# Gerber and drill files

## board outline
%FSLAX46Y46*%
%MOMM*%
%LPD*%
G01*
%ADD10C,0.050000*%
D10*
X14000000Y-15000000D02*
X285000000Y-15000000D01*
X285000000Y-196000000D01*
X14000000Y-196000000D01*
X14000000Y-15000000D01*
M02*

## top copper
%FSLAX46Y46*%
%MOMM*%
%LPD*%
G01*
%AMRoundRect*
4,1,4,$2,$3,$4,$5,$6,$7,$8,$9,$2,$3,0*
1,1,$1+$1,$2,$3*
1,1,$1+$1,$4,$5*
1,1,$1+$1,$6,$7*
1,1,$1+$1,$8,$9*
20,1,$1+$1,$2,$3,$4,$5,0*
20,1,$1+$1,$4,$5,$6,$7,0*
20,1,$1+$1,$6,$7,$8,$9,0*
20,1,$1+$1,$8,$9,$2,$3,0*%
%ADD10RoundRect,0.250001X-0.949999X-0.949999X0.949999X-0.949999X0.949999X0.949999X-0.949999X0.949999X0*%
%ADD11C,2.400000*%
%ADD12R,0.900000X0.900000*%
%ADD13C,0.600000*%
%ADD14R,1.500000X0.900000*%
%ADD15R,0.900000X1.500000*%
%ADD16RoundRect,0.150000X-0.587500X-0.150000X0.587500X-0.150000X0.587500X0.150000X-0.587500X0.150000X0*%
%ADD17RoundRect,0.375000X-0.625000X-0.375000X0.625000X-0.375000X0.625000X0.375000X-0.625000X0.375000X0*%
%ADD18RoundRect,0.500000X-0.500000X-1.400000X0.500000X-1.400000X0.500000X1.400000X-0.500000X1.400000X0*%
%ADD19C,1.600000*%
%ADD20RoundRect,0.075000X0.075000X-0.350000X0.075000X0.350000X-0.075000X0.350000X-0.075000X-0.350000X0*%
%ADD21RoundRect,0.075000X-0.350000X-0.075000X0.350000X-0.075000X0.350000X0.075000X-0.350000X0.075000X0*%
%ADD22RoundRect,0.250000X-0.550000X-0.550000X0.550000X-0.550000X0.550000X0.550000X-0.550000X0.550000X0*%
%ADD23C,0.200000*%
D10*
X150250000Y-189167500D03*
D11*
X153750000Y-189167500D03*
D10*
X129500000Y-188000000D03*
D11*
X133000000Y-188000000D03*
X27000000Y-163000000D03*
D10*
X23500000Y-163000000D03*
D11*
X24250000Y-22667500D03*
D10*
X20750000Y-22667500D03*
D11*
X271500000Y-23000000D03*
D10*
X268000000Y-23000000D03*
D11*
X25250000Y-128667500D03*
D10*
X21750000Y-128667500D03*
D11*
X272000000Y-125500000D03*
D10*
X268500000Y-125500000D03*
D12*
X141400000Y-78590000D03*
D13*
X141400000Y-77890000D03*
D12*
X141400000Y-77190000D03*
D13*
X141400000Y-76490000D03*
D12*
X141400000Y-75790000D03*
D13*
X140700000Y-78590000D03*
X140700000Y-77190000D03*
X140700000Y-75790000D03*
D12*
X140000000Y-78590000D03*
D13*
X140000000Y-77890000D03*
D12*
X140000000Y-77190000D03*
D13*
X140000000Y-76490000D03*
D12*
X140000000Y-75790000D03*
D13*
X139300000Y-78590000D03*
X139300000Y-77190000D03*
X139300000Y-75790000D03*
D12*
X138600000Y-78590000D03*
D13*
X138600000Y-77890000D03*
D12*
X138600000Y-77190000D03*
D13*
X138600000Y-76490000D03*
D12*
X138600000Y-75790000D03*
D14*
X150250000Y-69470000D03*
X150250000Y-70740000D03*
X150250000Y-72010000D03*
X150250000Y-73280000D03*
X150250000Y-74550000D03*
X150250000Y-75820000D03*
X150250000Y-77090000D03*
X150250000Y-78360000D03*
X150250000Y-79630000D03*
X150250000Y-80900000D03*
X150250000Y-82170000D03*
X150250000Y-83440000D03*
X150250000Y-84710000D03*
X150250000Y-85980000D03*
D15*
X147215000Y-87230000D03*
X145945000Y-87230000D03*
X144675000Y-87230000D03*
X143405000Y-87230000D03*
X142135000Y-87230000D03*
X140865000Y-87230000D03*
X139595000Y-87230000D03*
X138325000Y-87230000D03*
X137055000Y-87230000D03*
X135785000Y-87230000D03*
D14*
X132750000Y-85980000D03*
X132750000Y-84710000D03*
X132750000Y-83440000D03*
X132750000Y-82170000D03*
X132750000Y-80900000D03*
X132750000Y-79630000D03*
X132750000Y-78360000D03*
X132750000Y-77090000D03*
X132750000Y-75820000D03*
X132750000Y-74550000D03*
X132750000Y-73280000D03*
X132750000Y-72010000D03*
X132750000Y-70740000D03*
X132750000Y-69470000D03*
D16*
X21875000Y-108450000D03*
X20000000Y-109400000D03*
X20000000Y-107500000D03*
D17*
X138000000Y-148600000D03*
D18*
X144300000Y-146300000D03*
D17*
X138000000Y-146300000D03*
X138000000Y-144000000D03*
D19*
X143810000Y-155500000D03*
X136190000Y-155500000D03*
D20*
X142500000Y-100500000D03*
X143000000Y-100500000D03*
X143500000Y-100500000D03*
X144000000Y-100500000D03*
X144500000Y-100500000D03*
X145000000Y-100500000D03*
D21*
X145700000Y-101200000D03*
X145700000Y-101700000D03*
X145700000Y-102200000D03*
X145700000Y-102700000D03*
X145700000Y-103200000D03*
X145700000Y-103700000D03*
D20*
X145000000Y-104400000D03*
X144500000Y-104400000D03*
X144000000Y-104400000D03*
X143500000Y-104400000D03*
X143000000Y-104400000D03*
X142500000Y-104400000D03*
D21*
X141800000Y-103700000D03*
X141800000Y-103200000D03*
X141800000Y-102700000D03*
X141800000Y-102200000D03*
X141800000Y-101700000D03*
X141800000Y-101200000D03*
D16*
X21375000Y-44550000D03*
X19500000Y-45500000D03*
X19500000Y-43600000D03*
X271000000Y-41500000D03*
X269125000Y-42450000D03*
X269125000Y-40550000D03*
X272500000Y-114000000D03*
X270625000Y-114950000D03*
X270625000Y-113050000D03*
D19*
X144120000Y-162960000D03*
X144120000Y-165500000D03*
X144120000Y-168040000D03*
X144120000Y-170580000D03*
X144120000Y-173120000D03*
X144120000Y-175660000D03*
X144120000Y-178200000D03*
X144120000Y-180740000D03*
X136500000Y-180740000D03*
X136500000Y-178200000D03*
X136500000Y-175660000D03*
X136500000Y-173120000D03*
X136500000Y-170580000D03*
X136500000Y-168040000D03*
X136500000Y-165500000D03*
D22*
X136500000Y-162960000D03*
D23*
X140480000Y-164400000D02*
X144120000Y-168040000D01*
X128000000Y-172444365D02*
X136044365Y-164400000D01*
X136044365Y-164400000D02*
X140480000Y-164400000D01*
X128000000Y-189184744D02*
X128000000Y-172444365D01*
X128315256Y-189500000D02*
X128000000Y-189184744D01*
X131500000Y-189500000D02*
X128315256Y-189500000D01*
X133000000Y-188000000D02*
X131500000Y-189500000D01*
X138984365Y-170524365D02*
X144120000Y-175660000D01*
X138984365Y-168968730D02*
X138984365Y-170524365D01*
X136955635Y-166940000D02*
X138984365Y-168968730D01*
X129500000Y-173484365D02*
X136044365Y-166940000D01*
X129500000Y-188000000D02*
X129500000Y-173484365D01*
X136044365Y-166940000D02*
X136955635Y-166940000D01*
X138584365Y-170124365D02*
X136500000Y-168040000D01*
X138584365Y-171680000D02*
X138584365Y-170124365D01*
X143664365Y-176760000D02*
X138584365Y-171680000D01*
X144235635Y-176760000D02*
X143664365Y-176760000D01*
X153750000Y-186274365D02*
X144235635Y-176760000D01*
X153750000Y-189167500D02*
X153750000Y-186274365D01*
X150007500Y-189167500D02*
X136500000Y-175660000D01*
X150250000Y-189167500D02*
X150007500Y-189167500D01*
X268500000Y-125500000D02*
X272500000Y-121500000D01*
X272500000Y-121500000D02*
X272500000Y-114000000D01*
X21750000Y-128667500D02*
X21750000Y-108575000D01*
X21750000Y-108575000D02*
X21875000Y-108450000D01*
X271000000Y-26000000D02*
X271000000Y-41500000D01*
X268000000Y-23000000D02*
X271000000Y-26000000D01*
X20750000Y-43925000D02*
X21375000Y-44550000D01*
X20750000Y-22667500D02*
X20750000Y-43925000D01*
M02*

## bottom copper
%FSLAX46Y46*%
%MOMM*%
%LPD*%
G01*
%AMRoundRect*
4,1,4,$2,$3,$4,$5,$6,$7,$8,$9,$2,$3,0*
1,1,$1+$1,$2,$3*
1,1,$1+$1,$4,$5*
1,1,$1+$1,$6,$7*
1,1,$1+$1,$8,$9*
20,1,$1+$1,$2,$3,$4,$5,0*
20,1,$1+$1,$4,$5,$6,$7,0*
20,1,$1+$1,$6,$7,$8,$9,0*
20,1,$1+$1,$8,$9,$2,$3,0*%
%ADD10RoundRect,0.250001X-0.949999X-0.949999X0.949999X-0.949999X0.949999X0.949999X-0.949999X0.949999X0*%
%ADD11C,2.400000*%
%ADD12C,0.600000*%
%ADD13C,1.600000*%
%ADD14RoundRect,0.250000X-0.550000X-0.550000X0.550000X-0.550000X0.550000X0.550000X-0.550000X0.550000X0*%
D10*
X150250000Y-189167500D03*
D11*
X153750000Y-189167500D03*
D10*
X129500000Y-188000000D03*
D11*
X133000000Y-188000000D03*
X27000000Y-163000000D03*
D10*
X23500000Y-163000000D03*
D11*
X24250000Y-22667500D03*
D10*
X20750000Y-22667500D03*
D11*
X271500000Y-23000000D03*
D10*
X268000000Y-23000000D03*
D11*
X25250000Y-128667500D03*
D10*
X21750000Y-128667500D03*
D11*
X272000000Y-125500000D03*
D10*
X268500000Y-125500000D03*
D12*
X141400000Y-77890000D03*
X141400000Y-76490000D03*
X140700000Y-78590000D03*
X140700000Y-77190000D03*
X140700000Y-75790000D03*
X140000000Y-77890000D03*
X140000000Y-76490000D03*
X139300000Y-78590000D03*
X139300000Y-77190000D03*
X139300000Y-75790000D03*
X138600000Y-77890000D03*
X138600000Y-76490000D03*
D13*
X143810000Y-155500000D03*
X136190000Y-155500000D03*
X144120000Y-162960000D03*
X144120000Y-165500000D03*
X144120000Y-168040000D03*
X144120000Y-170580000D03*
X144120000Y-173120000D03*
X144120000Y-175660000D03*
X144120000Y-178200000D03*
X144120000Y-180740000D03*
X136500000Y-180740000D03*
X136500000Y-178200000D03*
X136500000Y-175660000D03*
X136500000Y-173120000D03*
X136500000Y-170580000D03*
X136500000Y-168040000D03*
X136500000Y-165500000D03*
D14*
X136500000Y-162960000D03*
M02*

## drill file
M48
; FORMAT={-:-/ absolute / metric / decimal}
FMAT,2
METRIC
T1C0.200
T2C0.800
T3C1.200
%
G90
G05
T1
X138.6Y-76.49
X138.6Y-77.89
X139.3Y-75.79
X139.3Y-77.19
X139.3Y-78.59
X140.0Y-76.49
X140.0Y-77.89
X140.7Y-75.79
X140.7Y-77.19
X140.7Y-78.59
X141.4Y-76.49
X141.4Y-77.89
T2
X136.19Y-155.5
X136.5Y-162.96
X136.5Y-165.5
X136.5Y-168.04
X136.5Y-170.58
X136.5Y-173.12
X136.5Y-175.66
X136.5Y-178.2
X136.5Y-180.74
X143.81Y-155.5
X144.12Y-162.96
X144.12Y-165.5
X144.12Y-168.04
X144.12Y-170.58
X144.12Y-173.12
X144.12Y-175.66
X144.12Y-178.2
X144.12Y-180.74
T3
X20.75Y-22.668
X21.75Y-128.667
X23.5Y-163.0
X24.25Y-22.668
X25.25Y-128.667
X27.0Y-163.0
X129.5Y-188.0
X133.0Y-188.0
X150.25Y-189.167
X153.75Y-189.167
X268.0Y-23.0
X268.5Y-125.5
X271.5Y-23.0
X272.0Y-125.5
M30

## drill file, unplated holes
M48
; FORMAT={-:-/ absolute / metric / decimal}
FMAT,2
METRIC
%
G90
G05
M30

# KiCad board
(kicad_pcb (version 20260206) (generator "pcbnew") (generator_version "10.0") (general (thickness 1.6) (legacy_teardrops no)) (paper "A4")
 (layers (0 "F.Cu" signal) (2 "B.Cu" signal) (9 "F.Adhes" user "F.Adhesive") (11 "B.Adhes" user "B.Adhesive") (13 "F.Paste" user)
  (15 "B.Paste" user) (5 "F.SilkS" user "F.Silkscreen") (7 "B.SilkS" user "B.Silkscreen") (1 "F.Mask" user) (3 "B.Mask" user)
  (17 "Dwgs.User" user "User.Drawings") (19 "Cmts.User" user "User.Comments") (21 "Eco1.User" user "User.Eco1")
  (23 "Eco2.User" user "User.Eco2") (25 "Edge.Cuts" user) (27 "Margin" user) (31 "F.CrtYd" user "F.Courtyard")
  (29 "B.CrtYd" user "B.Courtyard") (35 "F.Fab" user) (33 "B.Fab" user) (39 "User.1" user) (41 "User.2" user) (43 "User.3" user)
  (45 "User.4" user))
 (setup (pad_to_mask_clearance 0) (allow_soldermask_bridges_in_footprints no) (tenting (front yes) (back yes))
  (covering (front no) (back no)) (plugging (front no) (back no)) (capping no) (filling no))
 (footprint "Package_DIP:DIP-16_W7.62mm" (layer "F.Cu") (at 136.5 162.96)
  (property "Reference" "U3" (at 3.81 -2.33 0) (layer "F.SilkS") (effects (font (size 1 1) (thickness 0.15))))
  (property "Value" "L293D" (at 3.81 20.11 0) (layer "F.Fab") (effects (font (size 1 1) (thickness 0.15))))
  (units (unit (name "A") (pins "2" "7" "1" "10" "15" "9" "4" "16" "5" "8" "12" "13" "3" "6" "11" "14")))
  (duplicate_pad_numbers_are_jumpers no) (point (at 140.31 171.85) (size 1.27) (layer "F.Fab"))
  (pad "1" thru_hole roundrect (at 0 0) (size 1.6 1.6) (drill 0.8) (layers "*.Cu" "*.Mask") (remove_unused_layers no)
   (roundrect_rratio 0.15625) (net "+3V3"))
  (pad "2" thru_hole circle (at 0 2.54) (size 1.6 1.6) (drill 0.8) (layers "*.Cu" "*.Mask") (remove_unused_layers no) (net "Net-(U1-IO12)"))
  (pad "3" thru_hole circle (at 0 5.08) (size 1.6 1.6) (drill 0.8) (layers "*.Cu" "*.Mask") (remove_unused_layers no) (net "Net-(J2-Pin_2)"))
  (pad "4" thru_hole circle (at 0 7.62) (size 1.6 1.6) (drill 0.8) (layers "*.Cu" "*.Mask") (remove_unused_layers no) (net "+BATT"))
  (pad "5" thru_hole circle (at 0 10.16) (size 1.6 1.6) (drill 0.8) (layers "*.Cu" "*.Mask") (remove_unused_layers no) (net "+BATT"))
  (pad "6" thru_hole circle (at 0 12.7) (size 1.6 1.6) (drill 0.8) (layers "*.Cu" "*.Mask") (remove_unused_layers no) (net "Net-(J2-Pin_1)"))
  (pad "7" thru_hole circle (at 0 15.24) (size 1.6 1.6) (drill 0.8) (layers "*.Cu" "*.Mask") (remove_unused_layers no) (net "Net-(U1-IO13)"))
  (pad "8" thru_hole circle (at 0 17.78) (size 1.6 1.6) (drill 0.8) (layers "*.Cu" "*.Mask") (remove_unused_layers no) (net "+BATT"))
  (pad "9" thru_hole circle (at 7.62 17.78) (size 1.6 1.6) (drill 0.8) (layers "*.Cu" "*.Mask") (remove_unused_layers no) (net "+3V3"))
  (pad "10" thru_hole circle (at 7.62 15.24) (size 1.6 1.6) (drill 0.8) (layers "*.Cu" "*.Mask") (remove_unused_layers no)
   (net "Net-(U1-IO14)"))
  (pad "11" thru_hole circle (at 7.62 12.7) (size 1.6 1.6) (drill 0.8) (layers "*.Cu" "*.Mask") (remove_unused_layers no)
   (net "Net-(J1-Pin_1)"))
  (pad "12" thru_hole circle (at 7.62 10.16) (size 1.6 1.6) (drill 0.8) (layers "*.Cu" "*.Mask") (remove_unused_layers no) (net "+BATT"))
  (pad "13" thru_hole circle (at 7.62 7.62) (size 1.6 1.6) (drill 0.8) (layers "*.Cu" "*.Mask") (remove_unused_layers no) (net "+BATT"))
  (pad "14" thru_hole circle (at 7.62 5.08) (size 1.6 1.6) (drill 0.8) (layers "*.Cu" "*.Mask") (remove_unused_layers no)
   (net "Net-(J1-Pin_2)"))
  (pad "15" thru_hole circle (at 7.62 2.54) (size 1.6 1.6) (drill 0.8) (layers "*.Cu" "*.Mask") (remove_unused_layers no)
   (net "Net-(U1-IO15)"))
  (pad "16" thru_hole circle (at 7.62 0) (size 1.6 1.6) (drill 0.8) (layers "*.Cu" "*.Mask") (remove_unused_layers no)
   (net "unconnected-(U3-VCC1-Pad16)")))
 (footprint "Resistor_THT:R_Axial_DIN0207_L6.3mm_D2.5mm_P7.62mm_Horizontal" (layer "F.Cu") (at 136.19 155.5)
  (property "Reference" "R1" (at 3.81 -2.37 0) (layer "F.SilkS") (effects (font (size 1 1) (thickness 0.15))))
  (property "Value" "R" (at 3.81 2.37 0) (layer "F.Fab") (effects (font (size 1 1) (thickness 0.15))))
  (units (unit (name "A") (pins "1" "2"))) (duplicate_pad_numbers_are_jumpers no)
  (pad "1" thru_hole circle (at 0 0) (size 1.6 1.6) (drill 0.8) (layers "*.Cu" "*.Mask") (remove_unused_layers no) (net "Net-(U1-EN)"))
  (pad "2" thru_hole circle (at 7.62 0) (size 1.6 1.6) (drill 0.8) (layers "*.Cu" "*.Mask") (remove_unused_layers no) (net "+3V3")))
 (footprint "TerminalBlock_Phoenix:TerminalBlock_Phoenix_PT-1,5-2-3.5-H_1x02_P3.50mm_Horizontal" (layer "F.Cu") (at 268.5 125.5)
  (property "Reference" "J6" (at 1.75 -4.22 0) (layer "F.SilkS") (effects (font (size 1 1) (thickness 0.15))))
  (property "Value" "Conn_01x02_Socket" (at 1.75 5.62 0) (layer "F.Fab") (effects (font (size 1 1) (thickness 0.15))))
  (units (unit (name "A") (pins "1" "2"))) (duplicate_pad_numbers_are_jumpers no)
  (pad "1" thru_hole roundrect (at 0 0) (size 2.4 2.4) (drill 1.2) (layers "*.Cu" "*.Mask") (remove_unused_layers no)
   (roundrect_rratio 0.104167) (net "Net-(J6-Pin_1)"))
  (pad "2" thru_hole circle (at 3.5 0) (size 2.4 2.4) (drill 1.2) (layers "*.Cu" "*.Mask") (remove_unused_layers no) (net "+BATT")))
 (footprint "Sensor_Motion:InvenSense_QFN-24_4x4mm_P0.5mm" (layer "F.Cu") (at 143.75 102.45)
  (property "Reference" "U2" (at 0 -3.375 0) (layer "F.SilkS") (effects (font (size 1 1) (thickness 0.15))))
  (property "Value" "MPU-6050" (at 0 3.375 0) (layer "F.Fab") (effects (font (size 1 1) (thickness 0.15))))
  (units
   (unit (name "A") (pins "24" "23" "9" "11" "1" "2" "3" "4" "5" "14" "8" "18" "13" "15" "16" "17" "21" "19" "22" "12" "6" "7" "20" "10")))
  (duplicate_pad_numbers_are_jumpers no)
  (pad "1" smd roundrect (at -1.95 -1.25) (size 0.85 0.3) (layers "F.Cu" "F.Mask" "F.Paste") (roundrect_rratio 0.25)
   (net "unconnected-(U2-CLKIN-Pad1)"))
  (pad "2" smd roundrect (at -1.95 -0.75) (size 0.85 0.3) (layers "F.Cu" "F.Mask" "F.Paste") (roundrect_rratio 0.25)
   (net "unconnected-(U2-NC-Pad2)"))
  (pad "3" smd roundrect (at -1.95 -0.25) (size 0.85 0.3) (layers "F.Cu" "F.Mask" "F.Paste") (roundrect_rratio 0.25)
   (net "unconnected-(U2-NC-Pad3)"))
  (pad "4" smd roundrect (at -1.95 0.25) (size 0.85 0.3) (layers "F.Cu" "F.Mask" "F.Paste") (roundrect_rratio 0.25)
   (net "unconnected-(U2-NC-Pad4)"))
  (pad "5" smd roundrect (at -1.95 0.75) (size 0.85 0.3) (layers "F.Cu" "F.Mask" "F.Paste") (roundrect_rratio 0.25)
   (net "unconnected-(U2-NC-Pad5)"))
  (pad "6" smd roundrect (at -1.95 1.25) (size 0.85 0.3) (layers "F.Cu" "F.Mask" "F.Paste") (roundrect_rratio 0.25)
   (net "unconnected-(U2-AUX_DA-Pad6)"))
  (pad "7" smd roundrect (at -1.25 1.95 90) (size 0.85 0.3) (layers "F.Cu" "F.Mask" "F.Paste") (roundrect_rratio 0.25)
   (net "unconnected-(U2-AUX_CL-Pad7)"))
  (pad "8" smd roundrect (at -0.75 1.95 90) (size 0.85 0.3) (layers "F.Cu" "F.Mask" "F.Paste") (roundrect_rratio 0.25) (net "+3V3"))
  (pad "9" smd roundrect (at -0.25 1.95 90) (size 0.85 0.3) (layers "F.Cu" "F.Mask" "F.Paste") (roundrect_rratio 0.25)
   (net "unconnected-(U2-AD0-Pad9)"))
  (pad "10" smd roundrect (at 0.25 1.95 90) (size 0.85 0.3) (layers "F.Cu" "F.Mask" "F.Paste") (roundrect_rratio 0.25)
   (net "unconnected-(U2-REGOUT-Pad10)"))
  (pad "11" smd roundrect (at 0.75 1.95 90) (size 0.85 0.3) (layers "F.Cu" "F.Mask" "F.Paste") (roundrect_rratio 0.25)
   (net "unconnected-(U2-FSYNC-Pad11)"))
  (pad "12" smd roundrect (at 1.25 1.95 90) (size 0.85 0.3) (layers "F.Cu" "F.Mask" "F.Paste") (roundrect_rratio 0.25)
   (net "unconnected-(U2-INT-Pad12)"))
  (pad "13" smd roundrect (at 1.95 1.25) (size 0.85 0.3) (layers "F.Cu" "F.Mask" "F.Paste") (roundrect_rratio 0.25) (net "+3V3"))
  (pad "14" smd roundrect (at 1.95 0.75) (size 0.85 0.3) (layers "F.Cu" "F.Mask" "F.Paste") (roundrect_rratio 0.25)
   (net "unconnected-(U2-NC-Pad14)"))
  (pad "15" smd roundrect (at 1.95 0.25) (size 0.85 0.3) (layers "F.Cu" "F.Mask" "F.Paste") (roundrect_rratio 0.25)
   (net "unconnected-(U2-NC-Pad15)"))
  (pad "16" smd roundrect (at 1.95 -0.25) (size 0.85 0.3) (layers "F.Cu" "F.Mask" "F.Paste") (roundrect_rratio 0.25)
   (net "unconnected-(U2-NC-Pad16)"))
  (pad "17" smd roundrect (at 1.95 -0.75) (size 0.85 0.3) (layers "F.Cu" "F.Mask" "F.Paste") (roundrect_rratio 0.25)
   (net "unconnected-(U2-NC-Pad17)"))
  (pad "18" smd roundrect (at 1.95 -1.25) (size 0.85 0.3) (layers "F.Cu" "F.Mask" "F.Paste") (roundrect_rratio 0.25) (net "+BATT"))
  (pad "19" smd roundrect (at 1.25 -1.95 90) (size 0.85 0.3) (layers "F.Cu" "F.Mask" "F.Paste") (roundrect_rratio 0.25)
   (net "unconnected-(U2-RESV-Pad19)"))
  (pad "20" smd roundrect (at 0.75 -1.95 90) (size 0.85 0.3) (layers "F.Cu" "F.Mask" "F.Paste") (roundrect_rratio 0.25)
   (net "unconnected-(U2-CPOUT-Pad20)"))
  (pad "21" smd roundrect (at 0.25 -1.95 90) (size 0.85 0.3) (layers "F.Cu" "F.Mask" "F.Paste") (roundrect_rratio 0.25)
   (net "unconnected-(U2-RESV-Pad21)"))
  (pad "22" smd roundrect (at -0.25 -1.95 90) (size 0.85 0.3) (layers "F.Cu" "F.Mask" "F.Paste") (roundrect_rratio 0.25)
   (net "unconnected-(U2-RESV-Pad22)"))
  (pad "23" smd roundrect (at -0.75 -1.95 90) (size 0.85 0.3) (layers "F.Cu" "F.Mask" "F.Paste") (roundrect_rratio 0.25)
   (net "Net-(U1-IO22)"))
  (pad "24" smd roundrect (at -1.25 -1.95 90) (size 0.85 0.3) (layers "F.Cu" "F.Mask" "F.Paste") (roundrect_rratio 0.25)
   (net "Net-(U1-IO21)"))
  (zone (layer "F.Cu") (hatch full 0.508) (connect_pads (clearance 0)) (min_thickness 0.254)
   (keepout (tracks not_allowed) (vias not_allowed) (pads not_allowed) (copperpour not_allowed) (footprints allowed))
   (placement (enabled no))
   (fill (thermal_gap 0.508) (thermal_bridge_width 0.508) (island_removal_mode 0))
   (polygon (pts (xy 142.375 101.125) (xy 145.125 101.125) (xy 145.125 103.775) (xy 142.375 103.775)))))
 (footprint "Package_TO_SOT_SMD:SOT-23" (layer "F.Cu") (at 20.4375 44.55)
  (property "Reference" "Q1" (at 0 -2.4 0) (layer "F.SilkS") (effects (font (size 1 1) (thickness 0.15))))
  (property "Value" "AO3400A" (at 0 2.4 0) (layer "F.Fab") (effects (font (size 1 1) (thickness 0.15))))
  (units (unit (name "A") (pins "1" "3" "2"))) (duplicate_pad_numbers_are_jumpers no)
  (pad "1" smd roundrect (at -0.9375 -0.95) (size 1.475 0.6) (layers "F.Cu" "F.Mask" "F.Paste") (roundrect_rratio 0.25) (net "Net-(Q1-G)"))
  (pad "2" smd roundrect (at -0.9375 0.95) (size 1.475 0.6) (layers "F.Cu" "F.Mask" "F.Paste") (roundrect_rratio 0.25)
   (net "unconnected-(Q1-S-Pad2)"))
  (pad "3" smd roundrect (at 0.9375 0) (size 1.475 0.6) (layers "F.Cu" "F.Mask" "F.Paste") (roundrect_rratio 0.25) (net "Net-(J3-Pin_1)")))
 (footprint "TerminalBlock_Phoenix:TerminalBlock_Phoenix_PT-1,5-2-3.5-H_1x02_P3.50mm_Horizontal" (layer "F.Cu") (at 150.25 189.1675)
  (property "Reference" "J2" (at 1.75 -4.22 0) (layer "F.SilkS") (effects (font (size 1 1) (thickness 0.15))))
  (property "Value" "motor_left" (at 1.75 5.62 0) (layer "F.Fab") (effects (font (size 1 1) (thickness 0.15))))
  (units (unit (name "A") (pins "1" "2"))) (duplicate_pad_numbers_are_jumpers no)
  (pad "1" thru_hole roundrect (at 0 0) (size 2.4 2.4) (drill 1.2) (layers "*.Cu" "*.Mask") (remove_unused_layers no)
   (roundrect_rratio 0.104167) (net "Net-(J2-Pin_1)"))
  (pad "2" thru_hole circle (at 3.5 0) (size 2.4 2.4) (drill 1.2) (layers "*.Cu" "*.Mask") (remove_unused_layers no) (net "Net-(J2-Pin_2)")))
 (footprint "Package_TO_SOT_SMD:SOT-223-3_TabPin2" (layer "F.Cu") (at 141.15 146.3)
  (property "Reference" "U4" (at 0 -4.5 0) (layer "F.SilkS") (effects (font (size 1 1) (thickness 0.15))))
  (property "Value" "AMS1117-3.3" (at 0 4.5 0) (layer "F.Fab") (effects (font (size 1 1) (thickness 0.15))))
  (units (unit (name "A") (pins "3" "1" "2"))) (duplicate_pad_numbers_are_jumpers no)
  (pad "1" smd roundrect (at -3.15 -2.3) (size 2 1.5) (layers "F.Cu" "F.Mask" "F.Paste") (roundrect_rratio 0.25) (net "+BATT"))
  (pad "2" smd roundrect (at -3.15 0) (size 2 1.5) (layers "F.Cu" "F.Mask" "F.Paste") (roundrect_rratio 0.25) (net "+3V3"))
  (pad "2" smd roundrect (at 3.15 0) (size 2 3.8) (layers "F.Cu" "F.Mask" "F.Paste") (roundrect_rratio 0.25) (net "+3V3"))
  (pad "3" smd roundrect (at -3.15 2.3) (size 2 1.5) (layers "F.Cu" "F.Mask" "F.Paste") (roundrect_rratio 0.25) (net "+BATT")))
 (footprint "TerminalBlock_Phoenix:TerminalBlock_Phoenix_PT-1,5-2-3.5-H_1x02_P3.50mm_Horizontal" (layer "F.Cu") (at 23.5 163)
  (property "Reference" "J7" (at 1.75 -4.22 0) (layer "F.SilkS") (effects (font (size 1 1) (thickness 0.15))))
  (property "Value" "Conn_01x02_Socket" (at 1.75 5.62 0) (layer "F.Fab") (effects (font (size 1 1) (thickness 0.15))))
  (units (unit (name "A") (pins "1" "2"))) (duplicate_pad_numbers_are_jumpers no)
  (pad "1" thru_hole roundrect (at 0 0) (size 2.4 2.4) (drill 1.2) (layers "*.Cu" "*.Mask") (remove_unused_layers no)
   (roundrect_rratio 0.104167) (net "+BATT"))
  (pad "2" thru_hole circle (at 3.5 0) (size 2.4 2.4) (drill 1.2) (layers "*.Cu" "*.Mask") (remove_unused_layers no) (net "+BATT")))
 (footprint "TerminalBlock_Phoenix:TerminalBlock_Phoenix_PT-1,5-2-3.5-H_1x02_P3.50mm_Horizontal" (layer "F.Cu") (at 21.75 128.6675)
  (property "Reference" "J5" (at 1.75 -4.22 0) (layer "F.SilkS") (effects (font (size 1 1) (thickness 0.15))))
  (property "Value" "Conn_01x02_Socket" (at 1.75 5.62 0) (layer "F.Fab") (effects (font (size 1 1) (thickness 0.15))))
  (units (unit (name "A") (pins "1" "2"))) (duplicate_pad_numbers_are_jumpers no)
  (pad "1" thru_hole roundrect (at 0 0) (size 2.4 2.4) (drill 1.2) (layers "*.Cu" "*.Mask") (remove_unused_layers no)
   (roundrect_rratio 0.104167) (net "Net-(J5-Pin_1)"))
  (pad "2" thru_hole circle (at 3.5 0) (size 2.4 2.4) (drill 1.2) (layers "*.Cu" "*.Mask") (remove_unused_layers no) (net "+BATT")))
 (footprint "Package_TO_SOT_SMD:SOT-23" (layer "F.Cu") (at 20.9375 108.45)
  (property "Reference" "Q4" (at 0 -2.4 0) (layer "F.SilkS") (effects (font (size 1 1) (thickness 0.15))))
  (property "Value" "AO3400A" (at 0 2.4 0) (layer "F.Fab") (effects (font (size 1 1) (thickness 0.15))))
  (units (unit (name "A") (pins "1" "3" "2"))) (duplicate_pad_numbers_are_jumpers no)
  (pad "1" smd roundrect (at -0.9375 -0.95) (size 1.475 0.6) (layers "F.Cu" "F.Mask" "F.Paste") (roundrect_rratio 0.25) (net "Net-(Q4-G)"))
  (pad "2" smd roundrect (at -0.9375 0.95) (size 1.475 0.6) (layers "F.Cu" "F.Mask" "F.Paste") (roundrect_rratio 0.25)
   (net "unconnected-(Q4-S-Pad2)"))
  (pad "3" smd roundrect (at 0.9375 0) (size 1.475 0.6) (layers "F.Cu" "F.Mask" "F.Paste") (roundrect_rratio 0.25) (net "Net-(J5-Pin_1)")))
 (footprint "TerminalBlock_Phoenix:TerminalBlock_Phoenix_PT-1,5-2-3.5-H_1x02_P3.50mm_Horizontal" (layer "F.Cu") (at 268 23)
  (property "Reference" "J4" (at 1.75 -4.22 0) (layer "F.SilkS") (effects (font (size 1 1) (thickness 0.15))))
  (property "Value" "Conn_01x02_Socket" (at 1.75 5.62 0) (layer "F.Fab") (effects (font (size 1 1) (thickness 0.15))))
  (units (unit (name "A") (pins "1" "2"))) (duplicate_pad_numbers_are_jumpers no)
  (pad "1" thru_hole roundrect (at 0 0) (size 2.4 2.4) (drill 1.2) (layers "*.Cu" "*.Mask") (remove_unused_layers no)
   (roundrect_rratio 0.104167) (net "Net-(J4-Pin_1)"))
  (pad "2" thru_hole circle (at 3.5 0) (size 2.4 2.4) (drill 1.2) (layers "*.Cu" "*.Mask") (remove_unused_layers no) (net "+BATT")))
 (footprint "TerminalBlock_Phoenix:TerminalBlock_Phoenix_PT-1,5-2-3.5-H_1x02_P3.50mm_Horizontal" (layer "F.Cu") (at 129.5 188)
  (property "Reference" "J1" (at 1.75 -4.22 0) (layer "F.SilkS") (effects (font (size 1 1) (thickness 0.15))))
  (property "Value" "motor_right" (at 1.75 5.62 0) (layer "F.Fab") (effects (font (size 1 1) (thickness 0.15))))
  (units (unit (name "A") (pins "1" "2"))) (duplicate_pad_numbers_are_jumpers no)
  (pad "1" thru_hole roundrect (at 0 0) (size 2.4 2.4) (drill 1.2) (layers "*.Cu" "*.Mask") (remove_unused_layers no)
   (roundrect_rratio 0.104167) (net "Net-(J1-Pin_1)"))
  (pad "2" thru_hole circle (at 3.5 0) (size 2.4 2.4) (drill 1.2) (layers "*.Cu" "*.Mask") (remove_unused_layers no) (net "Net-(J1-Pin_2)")))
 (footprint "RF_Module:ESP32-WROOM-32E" (layer "F.Cu") (at 141.5 74.73)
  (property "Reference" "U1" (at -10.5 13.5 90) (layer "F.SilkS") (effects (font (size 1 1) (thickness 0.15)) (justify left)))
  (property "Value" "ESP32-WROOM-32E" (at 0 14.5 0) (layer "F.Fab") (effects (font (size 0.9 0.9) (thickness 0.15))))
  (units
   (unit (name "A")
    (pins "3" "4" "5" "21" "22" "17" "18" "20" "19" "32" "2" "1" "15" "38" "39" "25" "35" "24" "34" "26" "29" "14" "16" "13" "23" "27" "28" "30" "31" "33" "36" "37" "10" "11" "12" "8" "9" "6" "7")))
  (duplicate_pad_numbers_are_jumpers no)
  (pad "1" smd rect (at -8.75 -5.26) (size 1.5 0.9) (layers "F.Cu" "F.Mask" "F.Paste") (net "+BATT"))
  (pad "2" smd rect (at -8.75 -3.99) (size 1.5 0.9) (layers "F.Cu" "F.Mask" "F.Paste") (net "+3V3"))
  (pad "3" smd rect (at -8.75 -2.72) (size 1.5 0.9) (layers "F.Cu" "F.Mask" "F.Paste") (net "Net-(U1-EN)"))
  (pad "4" smd rect (at -8.75 -1.45) (size 1.5 0.9) (layers "F.Cu" "F.Mask" "F.Paste") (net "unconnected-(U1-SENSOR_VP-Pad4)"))
  (pad "5" smd rect (at -8.75 -0.18) (size 1.5 0.9) (layers "F.Cu" "F.Mask" "F.Paste") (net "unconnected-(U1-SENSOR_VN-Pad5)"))
  (pad "6" smd rect (at -8.75 1.09) (size 1.5 0.9) (layers "F.Cu" "F.Mask" "F.Paste") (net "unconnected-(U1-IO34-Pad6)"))
  (pad "7" smd rect (at -8.75 2.36) (size 1.5 0.9) (layers "F.Cu" "F.Mask" "F.Paste") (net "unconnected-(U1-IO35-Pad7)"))
  (pad "8" smd rect (at -8.75 3.63) (size 1.5 0.9) (layers "F.Cu" "F.Mask" "F.Paste") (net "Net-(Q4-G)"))
  (pad "9" smd rect (at -8.75 4.9) (size 1.5 0.9) (layers "F.Cu" "F.Mask" "F.Paste") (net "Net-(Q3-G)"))
  (pad "10" smd rect (at -8.75 6.17) (size 1.5 0.9) (layers "F.Cu" "F.Mask" "F.Paste") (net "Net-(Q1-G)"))
  (pad "11" smd rect (at -8.75 7.44) (size 1.5 0.9) (layers "F.Cu" "F.Mask" "F.Paste") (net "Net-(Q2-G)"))
  (pad "12" smd rect (at -8.75 8.71) (size 1.5 0.9) (layers "F.Cu" "F.Mask" "F.Paste") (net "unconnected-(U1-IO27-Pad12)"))
  (pad "13" smd rect (at -8.75 9.98) (size 1.5 0.9) (layers "F.Cu" "F.Mask" "F.Paste") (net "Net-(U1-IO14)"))
  (pad "14" smd rect (at -8.75 11.25) (size 1.5 0.9) (layers "F.Cu" "F.Mask" "F.Paste") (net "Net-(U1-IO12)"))
  (pad "15" smd rect (at -5.715 12.5 90) (size 1.5 0.9) (layers "F.Cu" "F.Mask" "F.Paste") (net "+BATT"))
  (pad "16" smd rect (at -4.445 12.5 90) (size 1.5 0.9) (layers "F.Cu" "F.Mask" "F.Paste") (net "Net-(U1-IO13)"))
  (pad "17" smd rect (at -3.175 12.5 90) (size 1.5 0.9) (layers "F.Cu" "F.Mask" "F.Paste") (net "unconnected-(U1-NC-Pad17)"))
  (pad "18" smd rect (at -1.905 12.5 90) (size 1.5 0.9) (layers "F.Cu" "F.Mask" "F.Paste") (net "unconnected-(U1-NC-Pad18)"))
  (pad "19" smd rect (at -0.635 12.5 90) (size 1.5 0.9) (layers "F.Cu" "F.Mask" "F.Paste") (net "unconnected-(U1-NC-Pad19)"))
  (pad "20" smd rect (at 0.635 12.5 90) (size 1.5 0.9) (layers "F.Cu" "F.Mask" "F.Paste") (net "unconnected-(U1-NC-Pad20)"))
  (pad "21" smd rect (at 1.905 12.5 90) (size 1.5 0.9) (layers "F.Cu" "F.Mask" "F.Paste") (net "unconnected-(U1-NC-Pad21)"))
  (pad "22" smd rect (at 3.175 12.5 90) (size 1.5 0.9) (layers "F.Cu" "F.Mask" "F.Paste") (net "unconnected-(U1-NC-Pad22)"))
  (pad "23" smd rect (at 4.445 12.5 90) (size 1.5 0.9) (layers "F.Cu" "F.Mask" "F.Paste") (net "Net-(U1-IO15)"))
  (pad "24" smd rect (at 5.715 12.5 90) (size 1.5 0.9) (layers "F.Cu" "F.Mask" "F.Paste") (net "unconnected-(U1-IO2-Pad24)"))
  (pad "25" smd rect (at 8.75 11.25) (size 1.5 0.9) (layers "F.Cu" "F.Mask" "F.Paste") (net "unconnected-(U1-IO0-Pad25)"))
  (pad "26" smd rect (at 8.75 9.98) (size 1.5 0.9) (layers "F.Cu" "F.Mask" "F.Paste") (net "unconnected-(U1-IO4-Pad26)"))
  (pad "27" smd rect (at 8.75 8.71) (size 1.5 0.9) (layers "F.Cu" "F.Mask" "F.Paste") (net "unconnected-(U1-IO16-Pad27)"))
  (pad "28" smd rect (at 8.75 7.44) (size 1.5 0.9) (layers "F.Cu" "F.Mask" "F.Paste") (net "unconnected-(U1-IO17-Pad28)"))
  (pad "29" smd rect (at 8.75 6.17) (size 1.5 0.9) (layers "F.Cu" "F.Mask" "F.Paste") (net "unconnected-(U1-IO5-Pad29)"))
  (pad "30" smd rect (at 8.75 4.9) (size 1.5 0.9) (layers "F.Cu" "F.Mask" "F.Paste") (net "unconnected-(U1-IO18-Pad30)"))
  (pad "31" smd rect (at 8.75 3.63) (size 1.5 0.9) (layers "F.Cu" "F.Mask" "F.Paste") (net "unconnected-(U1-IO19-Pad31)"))
  (pad "32" smd rect (at 8.75 2.36) (size 1.5 0.9) (layers "F.Cu" "F.Mask" "F.Paste") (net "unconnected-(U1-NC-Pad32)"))
  (pad "33" smd rect (at 8.75 1.09) (size 1.5 0.9) (layers "F.Cu" "F.Mask" "F.Paste") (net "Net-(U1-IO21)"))
  (pad "34" smd rect (at 8.75 -0.18) (size 1.5 0.9) (layers "F.Cu" "F.Mask" "F.Paste") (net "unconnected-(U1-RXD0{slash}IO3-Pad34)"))
  (pad "35" smd rect (at 8.75 -1.45) (size 1.5 0.9) (layers "F.Cu" "F.Mask" "F.Paste") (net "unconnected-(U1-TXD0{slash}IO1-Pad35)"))
  (pad "36" smd rect (at 8.75 -2.72) (size 1.5 0.9) (layers "F.Cu" "F.Mask" "F.Paste") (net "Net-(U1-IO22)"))
  (pad "37" smd rect (at 8.75 -3.99) (size 1.5 0.9) (layers "F.Cu" "F.Mask" "F.Paste") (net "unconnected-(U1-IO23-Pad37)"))
  (pad "38" smd rect (at 8.75 -5.26) (size 1.5 0.9) (layers "F.Cu" "F.Mask" "F.Paste") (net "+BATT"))
  (pad "39" smd rect (at -2.9 1.06) (size 0.9 0.9) (layers "F.Cu" "F.Mask" "F.Paste") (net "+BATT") (zone_connect 2))
  (pad "39" thru_hole circle (at -2.9 1.76) (size 0.6 0.6) (drill 0.2) (layers "*.Cu" "*.Mask") (remove_unused_layers no) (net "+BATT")
   (zone_connect 2))
  (pad "39" smd rect (at -2.9 2.46) (size 0.9 0.9) (layers "F.Cu" "F.Mask" "F.Paste") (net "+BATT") (zone_connect 2))
  (pad "39" thru_hole circle (at -2.9 3.16) (size 0.6 0.6) (drill 0.2) (layers "*.Cu" "*.Mask") (remove_unused_layers no) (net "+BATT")
   (zone_connect 2))
  (pad "39" smd rect (at -2.9 3.86) (size 0.9 0.9) (layers "F.Cu" "F.Mask" "F.Paste") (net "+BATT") (zone_connect 2))
  (pad "39" thru_hole circle (at -2.2 1.06) (size 0.6 0.6) (drill 0.2) (layers "*.Cu" "*.Mask") (remove_unused_layers no) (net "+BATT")
   (zone_connect 2))
  (pad "39" thru_hole circle (at -2.2 2.46) (size 0.6 0.6) (drill 0.2) (layers "*.Cu" "*.Mask") (remove_unused_layers no) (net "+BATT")
   (zone_connect 2))
  (pad "39" thru_hole circle (at -2.2 3.86) (size 0.6 0.6) (drill 0.2) (layers "*.Cu" "*.Mask") (remove_unused_layers no) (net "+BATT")
   (zone_connect 2))
  (pad "39" smd rect (at -1.5 1.06) (size 0.9 0.9) (layers "F.Cu" "F.Mask" "F.Paste") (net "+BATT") (zone_connect 2))
  (pad "39" thru_hole circle (at -1.5 1.76) (size 0.6 0.6) (drill 0.2) (layers "*.Cu" "*.Mask") (remove_unused_layers no) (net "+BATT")
   (zone_connect 2))
  (pad "39" smd rect (at -1.5 2.46) (size 0.9 0.9) (layers "F.Cu" "F.Mask" "F.Paste") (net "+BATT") (zone_connect 2))
  (pad "39" thru_hole circle (at -1.5 3.16) (size 0.6 0.6) (drill 0.2) (layers "*.Cu" "*.Mask") (remove_unused_layers no) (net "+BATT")
   (zone_connect 2))
  (pad "39" smd rect (at -1.5 3.86) (size 0.9 0.9) (layers "F.Cu" "F.Mask" "F.Paste") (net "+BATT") (zone_connect 2))
  (pad "39" thru_hole circle (at -0.8 1.06) (size 0.6 0.6) (drill 0.2) (layers "*.Cu" "*.Mask") (remove_unused_layers no) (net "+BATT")
   (zone_connect 2))
  (pad "39" thru_hole circle (at -0.8 2.46) (size 0.6 0.6) (drill 0.2) (layers "*.Cu" "*.Mask") (remove_unused_layers no) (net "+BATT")
   (zone_connect 2))
  (pad "39" thru_hole circle (at -0.8 3.86) (size 0.6 0.6) (drill 0.2) (layers "*.Cu" "*.Mask") (remove_unused_layers no) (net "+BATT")
   (zone_connect 2))
  (pad "39" smd rect (at -0.1 1.06) (size 0.9 0.9) (layers "F.Cu" "F.Mask" "F.Paste") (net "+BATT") (zone_connect 2))
  (pad "39" thru_hole circle (at -0.1 1.76) (size 0.6 0.6) (drill 0.2) (layers "*.Cu" "*.Mask") (remove_unused_layers no) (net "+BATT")
   (zone_connect 2))
  (pad "39" smd rect (at -0.1 2.46) (size 0.9 0.9) (layers "F.Cu" "F.Mask" "F.Paste") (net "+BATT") (zone_connect 2))
  (pad "39" thru_hole circle (at -0.1 3.16) (size 0.6 0.6) (drill 0.2) (layers "*.Cu" "*.Mask") (remove_unused_layers no) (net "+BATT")
   (zone_connect 2))
  (pad "39" smd rect (at -0.1 3.86) (size 0.9 0.9) (layers "F.Cu" "F.Mask" "F.Paste") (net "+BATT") (zone_connect 2))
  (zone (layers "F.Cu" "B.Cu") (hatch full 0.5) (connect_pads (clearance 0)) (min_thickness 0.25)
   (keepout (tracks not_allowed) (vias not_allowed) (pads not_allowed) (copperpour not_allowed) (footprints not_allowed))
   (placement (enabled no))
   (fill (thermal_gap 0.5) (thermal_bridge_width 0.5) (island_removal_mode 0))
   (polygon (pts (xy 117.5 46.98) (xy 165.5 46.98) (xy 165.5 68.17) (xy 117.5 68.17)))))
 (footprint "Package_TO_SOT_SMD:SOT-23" (layer "F.Cu") (at 271.5625 114)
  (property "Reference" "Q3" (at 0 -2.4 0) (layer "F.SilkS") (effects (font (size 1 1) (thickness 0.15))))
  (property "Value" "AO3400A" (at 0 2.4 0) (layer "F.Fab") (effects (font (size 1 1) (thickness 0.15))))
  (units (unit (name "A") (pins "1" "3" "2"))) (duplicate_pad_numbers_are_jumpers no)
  (pad "1" smd roundrect (at -0.9375 -0.95) (size 1.475 0.6) (layers "F.Cu" "F.Mask" "F.Paste") (roundrect_rratio 0.25) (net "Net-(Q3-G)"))
  (pad "2" smd roundrect (at -0.9375 0.95) (size 1.475 0.6) (layers "F.Cu" "F.Mask" "F.Paste") (roundrect_rratio 0.25)
   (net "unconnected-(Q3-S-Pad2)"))
  (pad "3" smd roundrect (at 0.9375 0) (size 1.475 0.6) (layers "F.Cu" "F.Mask" "F.Paste") (roundrect_rratio 0.25) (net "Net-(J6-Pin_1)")))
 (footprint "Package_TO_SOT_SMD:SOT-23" (layer "F.Cu") (at 270.0625 41.5)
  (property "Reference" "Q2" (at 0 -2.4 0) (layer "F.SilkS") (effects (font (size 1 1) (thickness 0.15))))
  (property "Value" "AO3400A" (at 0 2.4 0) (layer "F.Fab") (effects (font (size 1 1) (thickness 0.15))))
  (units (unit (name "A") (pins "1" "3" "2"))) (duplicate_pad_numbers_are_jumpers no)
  (pad "1" smd roundrect (at -0.9375 -0.95) (size 1.475 0.6) (layers "F.Cu" "F.Mask" "F.Paste") (roundrect_rratio 0.25) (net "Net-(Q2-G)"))
  (pad "2" smd roundrect (at -0.9375 0.95) (size 1.475 0.6) (layers "F.Cu" "F.Mask" "F.Paste") (roundrect_rratio 0.25)
   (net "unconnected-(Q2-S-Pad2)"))
  (pad "3" smd roundrect (at 0.9375 0) (size 1.475 0.6) (layers "F.Cu" "F.Mask" "F.Paste") (roundrect_rratio 0.25) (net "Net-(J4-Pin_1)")))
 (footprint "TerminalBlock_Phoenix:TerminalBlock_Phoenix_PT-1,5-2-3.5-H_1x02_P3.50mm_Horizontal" (layer "F.Cu") (at 20.75 22.6675)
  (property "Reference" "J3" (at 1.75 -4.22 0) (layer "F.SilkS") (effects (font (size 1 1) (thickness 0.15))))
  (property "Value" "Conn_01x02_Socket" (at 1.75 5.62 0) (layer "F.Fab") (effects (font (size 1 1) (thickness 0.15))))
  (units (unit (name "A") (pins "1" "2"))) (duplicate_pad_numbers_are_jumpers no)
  (pad "1" thru_hole roundrect (at 0 0) (size 2.4 2.4) (drill 1.2) (layers "*.Cu" "*.Mask") (remove_unused_layers no)
   (roundrect_rratio 0.104167) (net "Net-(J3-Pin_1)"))
  (pad "2" thru_hole circle (at 3.5 0) (size 2.4 2.4) (drill 1.2) (layers "*.Cu" "*.Mask") (remove_unused_layers no) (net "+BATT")))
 (gr_rect (start 14 15) (end 285 196) (stroke (width 0.05) (type default)) (fill no) (layer "Edge.Cuts"))
 (segment (start 136.044365 164.4) (end 140.48 164.4) (width 0.2) (layer "F.Cu") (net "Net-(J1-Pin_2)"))
 (segment (start 131.5 189.5) (end 128.315256 189.5) (width 0.2) (layer "F.Cu") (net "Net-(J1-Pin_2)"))
 (segment (start 128.315256 189.5) (end 128 189.184744) (width 0.2) (layer "F.Cu") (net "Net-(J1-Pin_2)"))
 (segment (start 140.48 164.4) (end 144.12 168.04) (width 0.2) (layer "F.Cu") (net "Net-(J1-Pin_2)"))
 (segment (start 128 172.444365) (end 136.044365 164.4) (width 0.2) (layer "F.Cu") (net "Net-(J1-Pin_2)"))
 (segment (start 128 189.184744) (end 128 172.444365) (width 0.2) (layer "F.Cu") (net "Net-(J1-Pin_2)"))
 (segment (start 133 188) (end 131.5 189.5) (width 0.2) (layer "F.Cu") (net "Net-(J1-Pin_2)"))
 (segment (start 138.984365 168.96873) (end 138.984365 170.524365) (width 0.2) (layer "F.Cu") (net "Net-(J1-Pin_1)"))
 (segment (start 138.984365 170.524365) (end 144.12 175.66) (width 0.2) (layer "F.Cu") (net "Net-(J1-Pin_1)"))
 (segment (start 129.5 173.484365) (end 136.044365 166.94) (width 0.2) (layer "F.Cu") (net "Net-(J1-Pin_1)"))
 (segment (start 136.955635 166.94) (end 138.984365 168.96873) (width 0.2) (layer "F.Cu") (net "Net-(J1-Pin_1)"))
 (segment (start 129.5 188) (end 129.5 173.484365) (width 0.2) (layer "F.Cu") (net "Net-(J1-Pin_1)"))
 (segment (start 136.044365 166.94) (end 136.955635 166.94) (width 0.2) (layer "F.Cu") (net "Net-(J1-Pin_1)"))
 (segment (start 143.664365 176.76) (end 138.584365 171.68) (width 0.2) (layer "F.Cu") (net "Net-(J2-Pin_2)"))
 (segment (start 138.584365 171.68) (end 138.584365 170.124365) (width 0.2) (layer "F.Cu") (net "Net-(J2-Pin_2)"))
 (segment (start 153.75 186.274365) (end 144.235635 176.76) (width 0.2) (layer "F.Cu") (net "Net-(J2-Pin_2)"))
 (segment (start 153.75 189.1675) (end 153.75 186.274365) (width 0.2) (layer "F.Cu") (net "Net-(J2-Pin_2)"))
 (segment (start 144.235635 176.76) (end 143.664365 176.76) (width 0.2) (layer "F.Cu") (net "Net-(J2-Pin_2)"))
 (segment (start 138.584365 170.124365) (end 136.5 168.04) (width 0.2) (layer "F.Cu") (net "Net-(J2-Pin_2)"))
 (segment (start 150.0075 189.1675) (end 136.5 175.66) (width 0.2) (layer "F.Cu") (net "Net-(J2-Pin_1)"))
 (segment (start 150.25 189.1675) (end 150.0075 189.1675) (width 0.2) (layer "F.Cu") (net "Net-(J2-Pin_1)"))
 (segment (start 20.75 43.925) (end 21.375 44.55) (width 0.2) (layer "F.Cu") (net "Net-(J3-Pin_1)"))
 (segment (start 20.75 22.6675) (end 20.75 43.925) (width 0.2) (layer "F.Cu") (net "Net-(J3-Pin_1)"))
 (segment (start 268 23) (end 271 26) (width 0.2) (layer "F.Cu") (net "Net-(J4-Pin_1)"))
 (segment (start 271 26) (end 271 41.5) (width 0.2) (layer "F.Cu") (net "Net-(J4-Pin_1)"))
 (segment (start 21.75 128.6675) (end 21.75 108.575) (width 0.2) (layer "F.Cu") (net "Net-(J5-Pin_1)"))
 (segment (start 21.75 108.575) (end 21.875 108.45) (width 0.2) (layer "F.Cu") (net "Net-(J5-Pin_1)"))
 (segment (start 268.5 125.5) (end 272.5 121.5) (width 0.2) (layer "F.Cu") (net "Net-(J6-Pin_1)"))
 (segment (start 272.5 121.5) (end 272.5 114) (width 0.2) (layer "F.Cu") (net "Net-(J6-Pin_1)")))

